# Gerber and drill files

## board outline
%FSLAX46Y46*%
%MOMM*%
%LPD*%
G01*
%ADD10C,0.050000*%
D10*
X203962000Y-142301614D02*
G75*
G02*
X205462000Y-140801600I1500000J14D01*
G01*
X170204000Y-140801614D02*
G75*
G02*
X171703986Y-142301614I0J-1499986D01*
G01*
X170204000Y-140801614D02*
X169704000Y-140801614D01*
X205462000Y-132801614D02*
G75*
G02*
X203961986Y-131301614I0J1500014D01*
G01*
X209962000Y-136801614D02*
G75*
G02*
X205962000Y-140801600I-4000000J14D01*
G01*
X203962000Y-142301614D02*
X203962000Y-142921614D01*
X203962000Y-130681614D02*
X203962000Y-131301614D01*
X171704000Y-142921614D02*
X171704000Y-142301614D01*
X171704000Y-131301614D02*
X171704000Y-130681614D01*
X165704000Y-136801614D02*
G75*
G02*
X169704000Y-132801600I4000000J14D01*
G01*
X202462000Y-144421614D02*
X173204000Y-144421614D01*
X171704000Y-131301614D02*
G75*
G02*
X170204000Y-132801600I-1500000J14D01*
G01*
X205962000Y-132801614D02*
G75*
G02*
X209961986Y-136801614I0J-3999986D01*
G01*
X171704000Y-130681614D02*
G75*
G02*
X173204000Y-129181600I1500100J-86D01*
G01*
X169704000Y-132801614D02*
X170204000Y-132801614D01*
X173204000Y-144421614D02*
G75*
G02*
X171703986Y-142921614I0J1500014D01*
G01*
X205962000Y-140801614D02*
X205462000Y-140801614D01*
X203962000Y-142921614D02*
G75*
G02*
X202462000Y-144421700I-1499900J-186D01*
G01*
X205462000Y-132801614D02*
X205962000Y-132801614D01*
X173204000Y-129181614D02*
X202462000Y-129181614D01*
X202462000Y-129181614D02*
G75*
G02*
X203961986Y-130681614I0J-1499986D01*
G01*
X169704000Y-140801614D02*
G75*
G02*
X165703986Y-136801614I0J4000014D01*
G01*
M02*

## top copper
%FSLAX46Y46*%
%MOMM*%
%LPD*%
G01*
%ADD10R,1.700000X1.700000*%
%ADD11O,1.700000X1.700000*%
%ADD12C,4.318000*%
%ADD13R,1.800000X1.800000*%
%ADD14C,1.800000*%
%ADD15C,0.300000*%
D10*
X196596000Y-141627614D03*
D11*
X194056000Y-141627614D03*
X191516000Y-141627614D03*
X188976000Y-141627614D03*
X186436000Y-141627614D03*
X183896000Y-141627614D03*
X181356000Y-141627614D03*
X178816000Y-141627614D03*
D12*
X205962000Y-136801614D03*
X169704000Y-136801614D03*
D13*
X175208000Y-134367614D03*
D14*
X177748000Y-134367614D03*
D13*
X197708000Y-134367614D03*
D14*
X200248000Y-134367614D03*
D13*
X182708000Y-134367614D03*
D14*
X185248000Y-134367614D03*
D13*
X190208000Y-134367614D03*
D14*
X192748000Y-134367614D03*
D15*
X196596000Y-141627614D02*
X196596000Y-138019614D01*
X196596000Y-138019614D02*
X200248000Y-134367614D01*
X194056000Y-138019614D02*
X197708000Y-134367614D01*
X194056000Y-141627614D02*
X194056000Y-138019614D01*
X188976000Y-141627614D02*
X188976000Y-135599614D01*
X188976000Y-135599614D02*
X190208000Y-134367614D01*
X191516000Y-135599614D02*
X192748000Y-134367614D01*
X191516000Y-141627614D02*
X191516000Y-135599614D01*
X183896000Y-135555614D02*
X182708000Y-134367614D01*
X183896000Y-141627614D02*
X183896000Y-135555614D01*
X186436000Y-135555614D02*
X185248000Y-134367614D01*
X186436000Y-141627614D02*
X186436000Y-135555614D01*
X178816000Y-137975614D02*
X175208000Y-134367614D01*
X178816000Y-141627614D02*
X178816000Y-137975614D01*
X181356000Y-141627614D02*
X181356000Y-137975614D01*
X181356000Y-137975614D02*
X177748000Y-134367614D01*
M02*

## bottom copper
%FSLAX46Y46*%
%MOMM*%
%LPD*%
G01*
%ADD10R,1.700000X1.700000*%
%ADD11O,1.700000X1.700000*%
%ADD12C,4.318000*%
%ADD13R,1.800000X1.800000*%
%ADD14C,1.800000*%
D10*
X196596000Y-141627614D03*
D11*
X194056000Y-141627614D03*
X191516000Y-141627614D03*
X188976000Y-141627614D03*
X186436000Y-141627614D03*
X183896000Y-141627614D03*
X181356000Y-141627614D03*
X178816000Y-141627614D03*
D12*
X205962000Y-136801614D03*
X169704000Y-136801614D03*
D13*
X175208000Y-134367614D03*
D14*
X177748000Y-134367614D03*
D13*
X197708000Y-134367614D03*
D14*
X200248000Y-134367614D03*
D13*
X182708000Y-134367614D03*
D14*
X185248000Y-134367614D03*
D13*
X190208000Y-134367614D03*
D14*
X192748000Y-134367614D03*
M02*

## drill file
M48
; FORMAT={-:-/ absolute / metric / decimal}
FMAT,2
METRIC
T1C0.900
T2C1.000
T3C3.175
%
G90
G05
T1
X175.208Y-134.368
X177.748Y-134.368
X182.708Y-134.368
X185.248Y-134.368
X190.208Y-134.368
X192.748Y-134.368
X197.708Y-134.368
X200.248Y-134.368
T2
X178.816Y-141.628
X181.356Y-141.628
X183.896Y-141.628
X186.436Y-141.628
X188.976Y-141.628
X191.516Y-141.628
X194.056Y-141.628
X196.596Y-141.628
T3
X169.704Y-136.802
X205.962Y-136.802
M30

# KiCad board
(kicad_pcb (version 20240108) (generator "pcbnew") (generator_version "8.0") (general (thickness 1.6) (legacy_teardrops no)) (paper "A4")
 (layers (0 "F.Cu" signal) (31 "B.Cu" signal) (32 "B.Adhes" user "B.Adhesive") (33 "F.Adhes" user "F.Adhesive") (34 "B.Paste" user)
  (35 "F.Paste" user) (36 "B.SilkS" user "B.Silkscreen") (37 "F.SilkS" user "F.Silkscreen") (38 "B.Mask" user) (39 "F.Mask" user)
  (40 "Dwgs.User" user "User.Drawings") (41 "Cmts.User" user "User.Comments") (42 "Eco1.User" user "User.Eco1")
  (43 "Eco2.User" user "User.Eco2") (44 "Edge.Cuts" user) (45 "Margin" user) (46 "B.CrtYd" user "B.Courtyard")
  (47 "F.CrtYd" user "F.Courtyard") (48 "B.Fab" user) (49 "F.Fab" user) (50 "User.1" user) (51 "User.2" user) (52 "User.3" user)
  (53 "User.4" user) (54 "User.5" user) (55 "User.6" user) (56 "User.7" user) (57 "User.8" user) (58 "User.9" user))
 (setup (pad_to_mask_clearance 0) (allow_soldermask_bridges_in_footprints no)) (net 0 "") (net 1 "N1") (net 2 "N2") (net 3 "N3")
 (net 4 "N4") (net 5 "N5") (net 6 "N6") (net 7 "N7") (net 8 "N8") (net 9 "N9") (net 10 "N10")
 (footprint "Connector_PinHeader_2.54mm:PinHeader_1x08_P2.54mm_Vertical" (layer "F.Cu") (at 196.596 141.627614 -90)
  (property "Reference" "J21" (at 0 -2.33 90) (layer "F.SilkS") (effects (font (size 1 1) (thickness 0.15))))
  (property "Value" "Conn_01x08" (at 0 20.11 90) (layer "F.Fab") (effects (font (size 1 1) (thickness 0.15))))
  (pad "1" thru_hole rect (at 0 0 270) (size 1.7 1.7) (drill 1) (layers "*.Cu" "*.Mask") (remove_unused_layers no) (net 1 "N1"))
  (pad "2" thru_hole oval (at 0 2.54 270) (size 1.7 1.7) (drill 1) (layers "*.Cu" "*.Mask") (remove_unused_layers no) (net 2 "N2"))
  (pad "3" thru_hole oval (at 0 5.08 270) (size 1.7 1.7) (drill 1) (layers "*.Cu" "*.Mask") (remove_unused_layers no) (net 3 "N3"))
  (pad "4" thru_hole oval (at 0 7.62 270) (size 1.7 1.7) (drill 1) (layers "*.Cu" "*.Mask") (remove_unused_layers no) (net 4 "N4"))
  (pad "5" thru_hole oval (at 0 10.16 270) (size 1.7 1.7) (drill 1) (layers "*.Cu" "*.Mask") (remove_unused_layers no) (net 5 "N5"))
  (pad "6" thru_hole oval (at 0 12.7 270) (size 1.7 1.7) (drill 1) (layers "*.Cu" "*.Mask") (remove_unused_layers no) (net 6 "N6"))
  (pad "7" thru_hole oval (at 0 15.24 270) (size 1.7 1.7) (drill 1) (layers "*.Cu" "*.Mask") (remove_unused_layers no) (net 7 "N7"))
  (pad "8" thru_hole oval (at 0 17.78 270) (size 1.7 1.7) (drill 1) (layers "*.Cu" "*.Mask") (remove_unused_layers no) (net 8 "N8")))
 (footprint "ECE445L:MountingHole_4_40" (layer "F.Cu") (at 205.962 136.801614 -90)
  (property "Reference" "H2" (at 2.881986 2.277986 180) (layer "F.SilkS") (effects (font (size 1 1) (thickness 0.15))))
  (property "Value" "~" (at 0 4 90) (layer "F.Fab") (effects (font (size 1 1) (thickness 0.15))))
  (pad "1" thru_hole circle (at 0 0 270) (size 4.318 4.318) (drill 3.175) (layers "*.Cu" "*.Mask") (remove_unused_layers no) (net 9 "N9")))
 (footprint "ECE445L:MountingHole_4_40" (layer "F.Cu") (at 169.704 136.801614 -90)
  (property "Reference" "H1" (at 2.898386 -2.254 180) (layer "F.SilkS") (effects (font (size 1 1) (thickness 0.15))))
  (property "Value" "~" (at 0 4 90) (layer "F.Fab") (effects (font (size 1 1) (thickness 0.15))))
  (pad "1" thru_hole circle (at 0 0 270) (size 4.318 4.318) (drill 3.175) (layers "*.Cu" "*.Mask") (remove_unused_layers no) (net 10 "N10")))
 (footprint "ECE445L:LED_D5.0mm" (layer "F.Cu") (at 175.208 134.367614)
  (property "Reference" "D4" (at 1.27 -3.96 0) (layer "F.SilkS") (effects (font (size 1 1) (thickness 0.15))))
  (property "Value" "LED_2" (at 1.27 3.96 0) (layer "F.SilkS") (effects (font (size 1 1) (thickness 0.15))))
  (pad "1" thru_hole rect (at 0 0) (size 1.8 1.8) (drill 0.9) (layers "*.Cu" "*.Mask") (remove_unused_layers no) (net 8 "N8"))
  (pad "2" thru_hole circle (at 2.54 0) (size 1.8 1.8) (drill 0.9) (layers "*.Cu" "*.Mask") (remove_unused_layers no) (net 7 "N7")))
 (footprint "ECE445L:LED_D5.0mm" (layer "F.Cu") (at 197.708 134.367614)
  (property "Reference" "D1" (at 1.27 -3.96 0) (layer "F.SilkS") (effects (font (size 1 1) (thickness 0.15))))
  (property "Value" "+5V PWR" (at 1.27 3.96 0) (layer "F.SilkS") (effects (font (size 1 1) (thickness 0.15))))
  (pad "1" thru_hole rect (at 0 0) (size 1.8 1.8) (drill 0.9) (layers "*.Cu" "*.Mask") (remove_unused_layers no) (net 2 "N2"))
  (pad "2" thru_hole circle (at 2.54 0) (size 1.8 1.8) (drill 0.9) (layers "*.Cu" "*.Mask") (remove_unused_layers no) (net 1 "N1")))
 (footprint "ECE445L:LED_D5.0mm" (layer "F.Cu") (at 182.708 134.367614)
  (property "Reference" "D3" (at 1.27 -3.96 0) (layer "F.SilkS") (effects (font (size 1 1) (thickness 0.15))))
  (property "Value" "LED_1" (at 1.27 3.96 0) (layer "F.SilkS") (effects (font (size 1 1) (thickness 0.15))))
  (pad "1" thru_hole rect (at 0 0) (size 1.8 1.8) (drill 0.9) (layers "*.Cu" "*.Mask") (remove_unused_layers no) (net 6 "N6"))
  (pad "2" thru_hole circle (at 2.54 0) (size 1.8 1.8) (drill 0.9) (layers "*.Cu" "*.Mask") (remove_unused_layers no) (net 5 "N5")))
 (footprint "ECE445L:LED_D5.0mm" (layer "F.Cu") (at 190.208 134.367614)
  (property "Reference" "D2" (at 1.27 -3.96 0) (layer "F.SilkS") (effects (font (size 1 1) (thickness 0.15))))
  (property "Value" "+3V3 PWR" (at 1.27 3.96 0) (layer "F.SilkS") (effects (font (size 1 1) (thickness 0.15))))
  (pad "1" thru_hole rect (at 0 0) (size 1.8 1.8) (drill 0.9) (layers "*.Cu" "*.Mask") (remove_unused_layers no) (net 4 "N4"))
  (pad "2" thru_hole circle (at 2.54 0) (size 1.8 1.8) (drill 0.9) (layers "*.Cu" "*.Mask") (remove_unused_layers no) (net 3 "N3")))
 (gr_arc (start 203.962 142.301614) (mid 204.401334 141.24094) (end 205.462 140.801614) (stroke (width 0.05) (type default))
  (layer "Edge.Cuts"))
 (gr_arc (start 170.204 140.801614) (mid 171.264664 141.24095) (end 171.704 142.301614) (stroke (width 0.05) (type default))
  (layer "Edge.Cuts"))
 (gr_line (start 170.204 140.801614) (end 169.704 140.801614) (stroke (width 0.05) (type default)) (layer "Edge.Cuts"))
 (gr_arc (start 205.462 132.801614) (mid 204.401344 132.36227) (end 203.962 131.301614) (stroke (width 0.05) (type default))
  (layer "Edge.Cuts"))
 (gr_arc (start 209.962 136.801614) (mid 208.790421 139.630027) (end 205.962 140.801614) (stroke (width 0.05) (type default))
  (layer "Edge.Cuts"))
 (gr_line (start 203.962 142.301614) (end 203.962 142.921614) (stroke (width 0.05) (type default)) (layer "Edge.Cuts"))
 (gr_line (start 203.962 130.681614) (end 203.962 131.301614) (stroke (width 0.05) (type default)) (layer "Edge.Cuts"))
 (gr_line (start 171.704 142.921614) (end 171.704 142.301614) (stroke (width 0.05) (type default)) (layer "Edge.Cuts"))
 (gr_line (start 171.704 131.301614) (end 171.704 130.681614) (stroke (width 0.05) (type default)) (layer "Edge.Cuts"))
 (gr_arc (start 165.704 136.801614) (mid 166.875567 133.973173) (end 169.704 132.801614) (stroke (width 0.05) (type default))
  (layer "Edge.Cuts"))
 (gr_line (start 202.462 144.421614) (end 173.204 144.421614) (stroke (width 0.05) (type default)) (layer "Edge.Cuts"))
 (gr_arc (start 171.704 131.301614) (mid 171.264654 132.36226) (end 170.204 132.801614) (stroke (width 0.05) (type default))
  (layer "Edge.Cuts"))
 (gr_arc (start 205.962 132.801614) (mid 208.790431 133.973183) (end 209.962 136.801614) (stroke (width 0.05) (type default))
  (layer "Edge.Cuts"))
 (gr_arc (start 171.704 130.681614) (mid 172.143369 129.621004) (end 173.204 129.181614) (stroke (width 0.05) (type default))
  (layer "Edge.Cuts"))
 (gr_line (start 169.704 132.801614) (end 170.204 132.801614) (stroke (width 0.05) (type default)) (layer "Edge.Cuts"))
 (gr_arc (start 173.204 144.421614) (mid 172.143344 143.98227) (end 171.704 142.921614) (stroke (width 0.05) (type default))
  (layer "Edge.Cuts"))
 (gr_line (start 205.962 140.801614) (end 205.462 140.801614) (stroke (width 0.05) (type default)) (layer "Edge.Cuts"))
 (gr_arc (start 203.962 142.921614) (mid 203.52269 143.982325) (end 202.462 144.421614) (stroke (width 0.05) (type default))
  (layer "Edge.Cuts"))
 (gr_line (start 205.462 132.801614) (end 205.962 132.801614) (stroke (width 0.05) (type default)) (layer "Edge.Cuts"))
 (gr_line (start 173.204 129.181614) (end 202.462 129.181614) (stroke (width 0.05) (type default)) (layer "Edge.Cuts"))
 (gr_arc (start 202.462 129.181614) (mid 203.522664 129.62095) (end 203.962 130.681614) (stroke (width 0.05) (type default))
  (layer "Edge.Cuts"))
 (gr_arc (start 169.704 140.801614) (mid 166.875577 139.630037) (end 165.704 136.801614) (stroke (width 0.05) (type default))
  (layer "Edge.Cuts"))
 (segment (start 196.596 141.627614) (end 196.596 138.019614) (width 0.3) (layer "F.Cu") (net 1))
 (segment (start 196.596 138.019614) (end 200.248 134.367614) (width 0.3) (layer "F.Cu") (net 1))
 (segment (start 194.056 138.019614) (end 197.708 134.367614) (width 0.3) (layer "F.Cu") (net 2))
 (segment (start 194.056 141.627614) (end 194.056 138.019614) (width 0.3) (layer "F.Cu") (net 2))
 (segment (start 188.976 141.627614) (end 188.976 135.599614) (width 0.3) (layer "F.Cu") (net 4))
 (segment (start 188.976 135.599614) (end 190.208 134.367614) (width 0.3) (layer "F.Cu") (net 4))
 (segment (start 191.516 135.599614) (end 192.748 134.367614) (width 0.3) (layer "F.Cu") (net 3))
 (segment (start 191.516 141.627614) (end 191.516 135.599614) (width 0.3) (layer "F.Cu") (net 3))
 (segment (start 183.896 135.555614) (end 182.708 134.367614) (width 0.3) (layer "F.Cu") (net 6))
 (segment (start 183.896 141.627614) (end 183.896 135.555614) (width 0.3) (layer "F.Cu") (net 6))
 (segment (start 186.436 135.555614) (end 185.248 134.367614) (width 0.3) (layer "F.Cu") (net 5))
 (segment (start 186.436 141.627614) (end 186.436 135.555614) (width 0.3) (layer "F.Cu") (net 5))
 (segment (start 178.816 137.975614) (end 175.208 134.367614) (width 0.3) (layer "F.Cu") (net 8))
 (segment (start 178.816 141.627614) (end 178.816 137.975614) (width 0.3) (layer "F.Cu") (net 8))
 (segment (start 181.356 141.627614) (end 181.356 137.975614) (width 0.3) (layer "F.Cu") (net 7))
 (segment (start 181.356 137.975614) (end 177.748 134.367614) (width 0.3) (layer "F.Cu") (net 7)))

